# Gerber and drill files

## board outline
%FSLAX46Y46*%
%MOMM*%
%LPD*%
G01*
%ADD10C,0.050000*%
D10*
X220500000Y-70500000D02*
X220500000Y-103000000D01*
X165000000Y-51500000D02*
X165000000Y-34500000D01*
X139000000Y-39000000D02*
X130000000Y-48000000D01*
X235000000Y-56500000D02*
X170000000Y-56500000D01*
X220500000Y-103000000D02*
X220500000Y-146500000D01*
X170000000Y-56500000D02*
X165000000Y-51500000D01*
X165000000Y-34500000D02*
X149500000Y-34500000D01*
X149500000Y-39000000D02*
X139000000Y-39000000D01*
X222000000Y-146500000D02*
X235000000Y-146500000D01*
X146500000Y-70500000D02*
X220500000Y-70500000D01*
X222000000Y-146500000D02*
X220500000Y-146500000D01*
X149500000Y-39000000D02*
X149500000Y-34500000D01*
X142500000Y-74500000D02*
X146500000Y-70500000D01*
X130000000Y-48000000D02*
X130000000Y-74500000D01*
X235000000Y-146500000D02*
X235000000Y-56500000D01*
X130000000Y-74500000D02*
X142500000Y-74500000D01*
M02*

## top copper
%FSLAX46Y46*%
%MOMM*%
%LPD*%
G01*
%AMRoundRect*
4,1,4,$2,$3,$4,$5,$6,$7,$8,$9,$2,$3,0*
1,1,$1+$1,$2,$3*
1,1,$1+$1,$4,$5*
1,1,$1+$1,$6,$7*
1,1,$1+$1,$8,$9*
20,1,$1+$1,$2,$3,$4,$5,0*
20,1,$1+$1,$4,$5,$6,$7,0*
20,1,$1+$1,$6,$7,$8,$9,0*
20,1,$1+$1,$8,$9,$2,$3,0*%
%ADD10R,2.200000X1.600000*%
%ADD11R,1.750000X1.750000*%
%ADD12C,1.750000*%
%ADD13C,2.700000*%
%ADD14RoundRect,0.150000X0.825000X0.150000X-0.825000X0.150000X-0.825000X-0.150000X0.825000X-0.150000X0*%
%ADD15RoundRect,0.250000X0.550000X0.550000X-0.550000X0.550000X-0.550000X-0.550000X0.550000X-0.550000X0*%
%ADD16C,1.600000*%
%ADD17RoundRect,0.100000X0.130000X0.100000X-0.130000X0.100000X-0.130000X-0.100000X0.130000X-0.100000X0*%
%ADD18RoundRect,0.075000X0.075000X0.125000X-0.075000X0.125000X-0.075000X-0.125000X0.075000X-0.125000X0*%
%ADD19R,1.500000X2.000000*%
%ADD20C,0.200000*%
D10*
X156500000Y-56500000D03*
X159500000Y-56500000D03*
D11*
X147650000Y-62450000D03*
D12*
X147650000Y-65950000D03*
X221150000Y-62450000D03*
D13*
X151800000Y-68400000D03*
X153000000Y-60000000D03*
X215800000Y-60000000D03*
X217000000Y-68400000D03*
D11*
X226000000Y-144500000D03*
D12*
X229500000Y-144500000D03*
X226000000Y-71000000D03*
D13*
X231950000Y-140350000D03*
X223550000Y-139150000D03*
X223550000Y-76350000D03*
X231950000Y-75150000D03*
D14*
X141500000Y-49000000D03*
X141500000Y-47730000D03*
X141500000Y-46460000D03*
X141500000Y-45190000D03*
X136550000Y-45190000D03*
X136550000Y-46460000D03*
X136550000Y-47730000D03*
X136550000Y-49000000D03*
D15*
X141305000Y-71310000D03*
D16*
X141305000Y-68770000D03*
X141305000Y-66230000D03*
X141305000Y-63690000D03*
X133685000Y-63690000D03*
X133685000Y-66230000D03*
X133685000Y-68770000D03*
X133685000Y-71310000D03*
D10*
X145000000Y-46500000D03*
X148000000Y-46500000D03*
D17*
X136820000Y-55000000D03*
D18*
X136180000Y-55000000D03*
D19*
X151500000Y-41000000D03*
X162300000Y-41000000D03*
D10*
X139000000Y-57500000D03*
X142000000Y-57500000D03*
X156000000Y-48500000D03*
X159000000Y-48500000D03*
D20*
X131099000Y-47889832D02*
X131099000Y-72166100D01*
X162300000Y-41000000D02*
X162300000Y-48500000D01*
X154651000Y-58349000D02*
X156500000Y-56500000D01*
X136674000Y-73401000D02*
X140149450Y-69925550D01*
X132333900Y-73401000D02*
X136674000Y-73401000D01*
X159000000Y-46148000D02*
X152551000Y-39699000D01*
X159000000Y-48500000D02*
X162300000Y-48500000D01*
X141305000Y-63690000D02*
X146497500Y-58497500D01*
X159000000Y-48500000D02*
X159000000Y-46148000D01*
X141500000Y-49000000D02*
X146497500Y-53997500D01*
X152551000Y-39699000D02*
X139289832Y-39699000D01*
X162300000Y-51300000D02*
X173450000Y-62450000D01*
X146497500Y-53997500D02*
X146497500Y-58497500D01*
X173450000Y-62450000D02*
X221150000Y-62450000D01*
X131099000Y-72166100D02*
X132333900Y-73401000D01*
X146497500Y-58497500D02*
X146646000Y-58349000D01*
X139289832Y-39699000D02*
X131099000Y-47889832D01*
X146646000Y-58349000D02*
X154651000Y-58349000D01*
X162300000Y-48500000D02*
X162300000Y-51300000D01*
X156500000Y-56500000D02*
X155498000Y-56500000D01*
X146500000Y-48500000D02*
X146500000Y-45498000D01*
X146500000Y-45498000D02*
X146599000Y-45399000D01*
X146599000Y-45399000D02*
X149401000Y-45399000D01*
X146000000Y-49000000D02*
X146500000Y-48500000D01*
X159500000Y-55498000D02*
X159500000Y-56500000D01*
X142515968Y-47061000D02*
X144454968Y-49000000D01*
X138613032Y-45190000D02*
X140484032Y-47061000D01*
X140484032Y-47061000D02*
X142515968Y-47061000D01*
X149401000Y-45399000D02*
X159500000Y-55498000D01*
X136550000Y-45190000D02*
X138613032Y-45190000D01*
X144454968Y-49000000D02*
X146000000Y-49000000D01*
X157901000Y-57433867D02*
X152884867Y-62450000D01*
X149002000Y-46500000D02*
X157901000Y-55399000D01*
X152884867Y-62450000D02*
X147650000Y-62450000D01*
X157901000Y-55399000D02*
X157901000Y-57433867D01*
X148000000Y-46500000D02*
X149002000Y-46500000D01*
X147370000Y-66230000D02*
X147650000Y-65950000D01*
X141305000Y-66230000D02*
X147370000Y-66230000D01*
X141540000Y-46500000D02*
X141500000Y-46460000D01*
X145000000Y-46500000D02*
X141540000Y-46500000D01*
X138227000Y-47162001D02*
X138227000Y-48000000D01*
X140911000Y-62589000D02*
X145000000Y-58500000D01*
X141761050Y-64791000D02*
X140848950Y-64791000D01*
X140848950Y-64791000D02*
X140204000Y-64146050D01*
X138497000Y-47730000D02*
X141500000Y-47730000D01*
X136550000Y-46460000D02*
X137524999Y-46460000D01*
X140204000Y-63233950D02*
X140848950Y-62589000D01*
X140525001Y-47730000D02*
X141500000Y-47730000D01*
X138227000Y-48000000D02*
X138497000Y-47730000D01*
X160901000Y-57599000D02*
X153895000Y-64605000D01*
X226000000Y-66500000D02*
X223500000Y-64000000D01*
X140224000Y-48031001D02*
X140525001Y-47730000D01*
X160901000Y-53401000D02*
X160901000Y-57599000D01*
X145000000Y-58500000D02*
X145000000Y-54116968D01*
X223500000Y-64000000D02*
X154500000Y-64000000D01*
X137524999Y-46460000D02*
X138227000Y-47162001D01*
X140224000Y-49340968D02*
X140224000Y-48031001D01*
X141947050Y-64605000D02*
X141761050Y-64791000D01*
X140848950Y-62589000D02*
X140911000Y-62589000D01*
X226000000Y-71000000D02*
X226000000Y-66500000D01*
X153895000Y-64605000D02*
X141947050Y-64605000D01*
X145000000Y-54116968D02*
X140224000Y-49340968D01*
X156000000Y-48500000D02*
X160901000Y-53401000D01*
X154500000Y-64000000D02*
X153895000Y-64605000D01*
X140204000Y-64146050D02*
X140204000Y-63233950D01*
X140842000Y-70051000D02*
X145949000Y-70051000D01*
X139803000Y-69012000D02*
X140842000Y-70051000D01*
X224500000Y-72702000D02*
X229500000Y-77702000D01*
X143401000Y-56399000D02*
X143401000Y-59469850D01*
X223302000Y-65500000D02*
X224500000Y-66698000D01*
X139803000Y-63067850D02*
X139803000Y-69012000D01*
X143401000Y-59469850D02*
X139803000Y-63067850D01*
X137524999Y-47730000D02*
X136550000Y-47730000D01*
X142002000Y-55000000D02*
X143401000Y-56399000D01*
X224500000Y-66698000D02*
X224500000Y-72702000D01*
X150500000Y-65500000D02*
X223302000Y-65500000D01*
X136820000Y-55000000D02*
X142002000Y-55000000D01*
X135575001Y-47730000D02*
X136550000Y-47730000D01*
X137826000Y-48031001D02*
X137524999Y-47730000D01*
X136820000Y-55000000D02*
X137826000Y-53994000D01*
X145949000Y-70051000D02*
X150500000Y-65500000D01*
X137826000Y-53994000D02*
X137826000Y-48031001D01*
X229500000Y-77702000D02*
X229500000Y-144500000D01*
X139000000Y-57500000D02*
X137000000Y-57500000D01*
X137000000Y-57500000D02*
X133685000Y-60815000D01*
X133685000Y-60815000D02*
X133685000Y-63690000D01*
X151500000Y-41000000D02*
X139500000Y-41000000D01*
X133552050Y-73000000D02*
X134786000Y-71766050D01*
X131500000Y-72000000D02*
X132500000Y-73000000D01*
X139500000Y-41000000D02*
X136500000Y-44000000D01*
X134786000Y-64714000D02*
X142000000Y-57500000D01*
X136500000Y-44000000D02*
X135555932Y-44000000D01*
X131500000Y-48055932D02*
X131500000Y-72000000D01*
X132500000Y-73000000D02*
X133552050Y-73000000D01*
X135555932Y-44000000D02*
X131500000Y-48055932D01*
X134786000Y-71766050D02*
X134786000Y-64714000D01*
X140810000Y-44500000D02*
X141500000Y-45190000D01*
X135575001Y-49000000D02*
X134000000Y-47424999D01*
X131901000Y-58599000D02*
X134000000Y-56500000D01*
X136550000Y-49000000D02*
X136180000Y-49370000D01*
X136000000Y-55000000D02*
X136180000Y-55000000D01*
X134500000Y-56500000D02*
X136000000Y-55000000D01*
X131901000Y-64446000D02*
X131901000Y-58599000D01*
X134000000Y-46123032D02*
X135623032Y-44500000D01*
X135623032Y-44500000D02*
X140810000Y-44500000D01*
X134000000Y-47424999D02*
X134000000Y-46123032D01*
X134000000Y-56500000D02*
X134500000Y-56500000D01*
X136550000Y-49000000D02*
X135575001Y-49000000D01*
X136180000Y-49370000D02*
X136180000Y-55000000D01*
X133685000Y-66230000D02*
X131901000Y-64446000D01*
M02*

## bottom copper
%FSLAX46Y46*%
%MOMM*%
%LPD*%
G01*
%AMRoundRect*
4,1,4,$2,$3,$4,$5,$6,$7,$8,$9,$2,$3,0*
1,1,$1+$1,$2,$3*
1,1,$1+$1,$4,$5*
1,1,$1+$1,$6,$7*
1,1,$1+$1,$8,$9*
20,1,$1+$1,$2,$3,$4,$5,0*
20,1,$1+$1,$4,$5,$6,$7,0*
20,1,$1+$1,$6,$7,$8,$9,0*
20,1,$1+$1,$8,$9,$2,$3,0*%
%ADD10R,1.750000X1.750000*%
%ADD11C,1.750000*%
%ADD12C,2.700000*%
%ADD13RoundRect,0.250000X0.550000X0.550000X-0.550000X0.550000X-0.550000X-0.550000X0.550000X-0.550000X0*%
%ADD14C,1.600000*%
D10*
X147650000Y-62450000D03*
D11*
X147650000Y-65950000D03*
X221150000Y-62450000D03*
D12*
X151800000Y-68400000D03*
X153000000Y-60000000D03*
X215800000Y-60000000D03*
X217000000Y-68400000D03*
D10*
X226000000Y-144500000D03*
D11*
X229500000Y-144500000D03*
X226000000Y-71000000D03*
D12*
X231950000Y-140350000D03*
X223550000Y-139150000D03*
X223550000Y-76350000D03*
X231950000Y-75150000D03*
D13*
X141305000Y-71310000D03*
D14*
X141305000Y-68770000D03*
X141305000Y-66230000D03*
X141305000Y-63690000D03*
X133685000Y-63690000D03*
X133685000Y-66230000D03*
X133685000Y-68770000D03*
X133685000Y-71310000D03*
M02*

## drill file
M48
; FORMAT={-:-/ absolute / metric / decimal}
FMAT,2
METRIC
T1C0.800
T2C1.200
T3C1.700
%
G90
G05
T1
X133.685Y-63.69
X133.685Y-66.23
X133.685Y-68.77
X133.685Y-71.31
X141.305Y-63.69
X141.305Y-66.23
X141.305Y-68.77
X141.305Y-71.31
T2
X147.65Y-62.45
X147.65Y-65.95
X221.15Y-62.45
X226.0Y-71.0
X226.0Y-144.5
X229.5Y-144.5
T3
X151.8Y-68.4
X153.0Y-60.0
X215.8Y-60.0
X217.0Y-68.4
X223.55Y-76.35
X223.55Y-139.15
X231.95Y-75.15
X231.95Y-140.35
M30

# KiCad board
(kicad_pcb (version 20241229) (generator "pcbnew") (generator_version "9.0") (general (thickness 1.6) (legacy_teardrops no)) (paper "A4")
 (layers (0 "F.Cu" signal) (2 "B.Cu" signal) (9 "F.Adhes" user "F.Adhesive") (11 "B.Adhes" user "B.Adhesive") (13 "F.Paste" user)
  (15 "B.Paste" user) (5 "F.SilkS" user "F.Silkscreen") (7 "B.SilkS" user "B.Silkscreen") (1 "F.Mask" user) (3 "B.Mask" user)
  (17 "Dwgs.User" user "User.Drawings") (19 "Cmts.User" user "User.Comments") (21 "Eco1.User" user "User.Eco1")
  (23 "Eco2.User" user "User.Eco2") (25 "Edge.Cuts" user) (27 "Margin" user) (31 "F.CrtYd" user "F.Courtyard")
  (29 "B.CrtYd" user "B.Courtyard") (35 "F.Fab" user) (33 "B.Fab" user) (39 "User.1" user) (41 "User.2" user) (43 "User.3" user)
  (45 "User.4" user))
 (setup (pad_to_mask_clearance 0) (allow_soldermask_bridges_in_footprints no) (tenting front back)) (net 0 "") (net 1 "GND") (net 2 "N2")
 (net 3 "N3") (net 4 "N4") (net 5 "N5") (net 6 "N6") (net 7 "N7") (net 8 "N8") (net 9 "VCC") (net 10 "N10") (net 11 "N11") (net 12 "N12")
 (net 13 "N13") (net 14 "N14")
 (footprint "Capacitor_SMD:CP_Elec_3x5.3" (layer "F.Cu") (at 158 56.5)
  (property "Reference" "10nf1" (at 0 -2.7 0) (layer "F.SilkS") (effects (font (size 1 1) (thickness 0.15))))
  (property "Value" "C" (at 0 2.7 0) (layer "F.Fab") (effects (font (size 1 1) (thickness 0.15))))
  (pad "1" smd rect (at -1.5 0) (size 2.2 1.6) (layers "F.Cu" "F.Mask" "F.Paste") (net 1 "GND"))
  (pad "2" smd rect (at 1.5 0) (size 2.2 1.6) (layers "F.Cu" "F.Mask" "F.Paste") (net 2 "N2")))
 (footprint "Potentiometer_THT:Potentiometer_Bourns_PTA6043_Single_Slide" (layer "F.Cu") (at 147.65 62.45)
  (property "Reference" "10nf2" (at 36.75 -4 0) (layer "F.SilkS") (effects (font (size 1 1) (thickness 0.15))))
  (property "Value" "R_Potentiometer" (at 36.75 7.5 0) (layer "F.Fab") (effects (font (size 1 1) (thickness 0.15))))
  (pad "1" thru_hole rect (at 0 0) (size 1.75 1.75) (drill 1.2) (layers "*.Cu" "*.Mask") (remove_unused_layers no) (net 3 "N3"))
  (pad "2" thru_hole circle (at 0 3.5) (size 1.75 1.75) (drill 1.2) (layers "*.Cu" "*.Mask") (remove_unused_layers no) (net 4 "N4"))
  (pad "3" thru_hole circle (at 73.5 0) (size 1.75 1.75) (drill 1.2) (layers "*.Cu" "*.Mask") (remove_unused_layers no) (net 1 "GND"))
  (pad "MP" thru_hole circle (at 4.15 5.95) (size 2.7 2.7) (drill 1.7) (layers "*.Cu" "*.Mask") (remove_unused_layers no))
  (pad "MP" thru_hole circle (at 5.35 -2.45) (size 2.7 2.7) (drill 1.7) (layers "*.Cu" "*.Mask") (remove_unused_layers no))
  (pad "MP" thru_hole circle (at 68.15 -2.45) (size 2.7 2.7) (drill 1.7) (layers "*.Cu" "*.Mask") (remove_unused_layers no))
  (pad "MP" thru_hole circle (at 69.35 5.95) (size 2.7 2.7) (drill 1.7) (layers "*.Cu" "*.Mask") (remove_unused_layers no)))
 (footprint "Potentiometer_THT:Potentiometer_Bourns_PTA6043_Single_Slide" (layer "F.Cu") (at 226 144.5 90)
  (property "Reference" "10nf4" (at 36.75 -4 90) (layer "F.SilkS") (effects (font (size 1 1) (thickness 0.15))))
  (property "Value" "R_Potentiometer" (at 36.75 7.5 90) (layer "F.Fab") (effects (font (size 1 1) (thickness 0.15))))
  (pad "1" thru_hole rect (at 0 0 90) (size 1.75 1.75) (drill 1.2) (layers "*.Cu" "*.Mask") (remove_unused_layers no) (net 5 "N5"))
  (pad "2" thru_hole circle (at 0 3.5 90) (size 1.75 1.75) (drill 1.2) (layers "*.Cu" "*.Mask") (remove_unused_layers no) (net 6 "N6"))
  (pad "3" thru_hole circle (at 73.5 0 90) (size 1.75 1.75) (drill 1.2) (layers "*.Cu" "*.Mask") (remove_unused_layers no) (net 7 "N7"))
  (pad "MP" thru_hole circle (at 4.15 5.95 90) (size 2.7 2.7) (drill 1.7) (layers "*.Cu" "*.Mask") (remove_unused_layers no))
  (pad "MP" thru_hole circle (at 5.35 -2.45 90) (size 2.7 2.7) (drill 1.7) (layers "*.Cu" "*.Mask") (remove_unused_layers no))
  (pad "MP" thru_hole circle (at 68.15 -2.45 90) (size 2.7 2.7) (drill 1.7) (layers "*.Cu" "*.Mask") (remove_unused_layers no))
  (pad "MP" thru_hole circle (at 69.35 5.95 90) (size 2.7 2.7) (drill 1.7) (layers "*.Cu" "*.Mask") (remove_unused_layers no)))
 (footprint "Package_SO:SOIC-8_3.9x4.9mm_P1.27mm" (layer "F.Cu") (at 139.025 47.095 180)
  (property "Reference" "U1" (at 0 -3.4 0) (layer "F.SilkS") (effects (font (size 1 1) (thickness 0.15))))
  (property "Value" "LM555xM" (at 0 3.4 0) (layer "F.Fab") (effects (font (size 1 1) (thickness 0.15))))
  (pad "1" smd roundrect (at -2.475 -1.905 180) (size 1.95 0.6) (layers "F.Cu" "F.Mask" "F.Paste") (roundrect_rratio 0.25) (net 1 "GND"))
  (pad "2" smd roundrect (at -2.475 -0.635 180) (size 1.95 0.6) (layers "F.Cu" "F.Mask" "F.Paste") (roundrect_rratio 0.25) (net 7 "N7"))
  (pad "3" smd roundrect (at -2.475 0.635 180) (size 1.95 0.6) (layers "F.Cu" "F.Mask" "F.Paste") (roundrect_rratio 0.25) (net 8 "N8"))
  (pad "4" smd roundrect (at -2.475 1.905 180) (size 1.95 0.6) (layers "F.Cu" "F.Mask" "F.Paste") (roundrect_rratio 0.25) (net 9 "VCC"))
  (pad "5" smd roundrect (at 2.475 1.905 180) (size 1.95 0.6) (layers "F.Cu" "F.Mask" "F.Paste") (roundrect_rratio 0.25) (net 2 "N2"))
  (pad "6" smd roundrect (at 2.475 0.635 180) (size 1.95 0.6) (layers "F.Cu" "F.Mask" "F.Paste") (roundrect_rratio 0.25) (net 7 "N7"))
  (pad "7" smd roundrect (at 2.475 -0.635 180) (size 1.95 0.6) (layers "F.Cu" "F.Mask" "F.Paste") (roundrect_rratio 0.25) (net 6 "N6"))
  (pad "8" smd roundrect (at 2.475 -1.905 180) (size 1.95 0.6) (layers "F.Cu" "F.Mask" "F.Paste") (roundrect_rratio 0.25) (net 9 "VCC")))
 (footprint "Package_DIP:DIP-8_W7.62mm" (layer "F.Cu") (at 141.305 71.31 180)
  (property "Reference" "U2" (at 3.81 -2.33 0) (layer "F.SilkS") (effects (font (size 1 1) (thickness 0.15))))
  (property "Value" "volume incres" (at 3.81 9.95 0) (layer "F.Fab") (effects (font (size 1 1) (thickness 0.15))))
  (pad "1" thru_hole roundrect (at 0 0 180) (size 1.6 1.6) (drill 0.8) (layers "*.Cu" "*.Mask") (remove_unused_layers no)
   (roundrect_rratio 0.15625) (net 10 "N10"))
  (pad "2" thru_hole circle (at 0 2.54 180) (size 1.6 1.6) (drill 0.8) (layers "*.Cu" "*.Mask") (remove_unused_layers no) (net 1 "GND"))
  (pad "3" thru_hole circle (at 0 5.08 180) (size 1.6 1.6) (drill 0.8) (layers "*.Cu" "*.Mask") (remove_unused_layers no) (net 4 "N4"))
  (pad "4" thru_hole circle (at 0 7.62 180) (size 1.6 1.6) (drill 0.8) (layers "*.Cu" "*.Mask") (remove_unused_layers no) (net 1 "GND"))
  (pad "5" thru_hole circle (at 7.62 7.62 180) (size 1.6 1.6) (drill 0.8) (layers "*.Cu" "*.Mask") (remove_unused_layers no) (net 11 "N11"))
  (pad "6" thru_hole circle (at 7.62 5.08 180) (size 1.6 1.6) (drill 0.8) (layers "*.Cu" "*.Mask") (remove_unused_layers no) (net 9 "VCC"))
  (pad "7" thru_hole circle (at 7.62 2.54 180) (size 1.6 1.6) (drill 0.8) (layers "*.Cu" "*.Mask") (remove_unused_layers no) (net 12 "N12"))
  (pad "8" thru_hole circle (at 7.62 0 180) (size 1.6 1.6) (drill 0.8) (layers "*.Cu" "*.Mask") (remove_unused_layers no) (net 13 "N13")))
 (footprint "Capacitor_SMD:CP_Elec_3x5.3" (layer "F.Cu") (at 146.5 46.5)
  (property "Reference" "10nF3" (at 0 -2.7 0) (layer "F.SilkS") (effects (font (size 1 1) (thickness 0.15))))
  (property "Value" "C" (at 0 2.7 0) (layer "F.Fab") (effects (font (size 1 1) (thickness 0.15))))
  (pad "1" smd rect (at -1.5 0) (size 2.2 1.6) (layers "F.Cu" "F.Mask" "F.Paste") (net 8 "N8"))
  (pad "2" smd rect (at 1.5 0) (size 2.2 1.6) (layers "F.Cu" "F.Mask" "F.Paste") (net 3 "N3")))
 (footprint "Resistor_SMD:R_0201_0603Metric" (layer "F.Cu") (at 136.5 55 180)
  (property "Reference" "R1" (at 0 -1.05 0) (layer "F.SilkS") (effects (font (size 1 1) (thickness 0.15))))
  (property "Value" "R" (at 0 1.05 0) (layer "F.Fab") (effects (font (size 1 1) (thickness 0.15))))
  (pad "" smd roundrect (at -0.345 0 180) (size 0.318 0.36) (layers "F.Paste") (roundrect_rratio 0.25))
  (pad "" smd roundrect (at 0.345 0 180) (size 0.318 0.36) (layers "F.Paste") (roundrect_rratio 0.25))
  (pad "1" smd roundrect (at -0.32 0 180) (size 0.46 0.4) (layers "F.Cu" "F.Mask") (roundrect_rratio 0.25) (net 6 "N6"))
  (pad "2" smd roundrect (at 0.32 0 180) (size 0.3 0.4) (layers "F.Cu" "F.Mask") (roundrect_rratio 0.25) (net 9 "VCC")))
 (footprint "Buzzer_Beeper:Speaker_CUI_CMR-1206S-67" (layer "F.Cu") (at 156.9 38.7)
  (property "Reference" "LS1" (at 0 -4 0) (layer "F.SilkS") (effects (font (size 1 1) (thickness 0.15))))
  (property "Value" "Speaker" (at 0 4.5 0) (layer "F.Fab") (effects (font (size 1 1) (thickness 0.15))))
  (pad "1" smd rect (at -5.4 2.3 180) (size 1.5 2) (layers "F.Cu" "F.Mask") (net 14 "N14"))
  (pad "2" smd rect (at 5.4 2.3 180) (size 1.5 2) (layers "F.Cu" "F.Mask") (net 1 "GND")))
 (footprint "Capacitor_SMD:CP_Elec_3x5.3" (layer "F.Cu") (at 140.5 57.5)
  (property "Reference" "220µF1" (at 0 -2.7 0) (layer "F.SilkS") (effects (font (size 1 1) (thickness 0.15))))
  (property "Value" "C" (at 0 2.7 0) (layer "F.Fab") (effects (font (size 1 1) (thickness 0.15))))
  (pad "1" smd rect (at -1.5 0) (size 2.2 1.6) (layers "F.Cu" "F.Mask" "F.Paste") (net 11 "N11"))
  (pad "2" smd rect (at 1.5 0) (size 2.2 1.6) (layers "F.Cu" "F.Mask" "F.Paste") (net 14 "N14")))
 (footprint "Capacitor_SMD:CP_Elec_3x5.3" (layer "F.Cu") (at 157.5 48.5)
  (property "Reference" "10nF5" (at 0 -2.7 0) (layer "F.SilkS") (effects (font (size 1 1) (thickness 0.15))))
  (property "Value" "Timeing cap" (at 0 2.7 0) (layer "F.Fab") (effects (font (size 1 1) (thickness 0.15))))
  (pad "1" smd rect (at -1.5 0) (size 2.2 1.6) (layers "F.Cu" "F.Mask" "F.Paste") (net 7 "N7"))
  (pad "2" smd rect (at 1.5 0) (size 2.2 1.6) (layers "F.Cu" "F.Mask" "F.Paste") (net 1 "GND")))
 (gr_line (start 220.5 70.5) (end 220.5 103) (stroke (width 0.05) (type default)) (layer "Edge.Cuts"))
 (gr_line (start 165 51.5) (end 165 34.5) (stroke (width 0.05) (type default)) (layer "Edge.Cuts"))
 (gr_line (start 139 39) (end 130 48) (stroke (width 0.05) (type default)) (layer "Edge.Cuts"))
 (gr_line (start 235 56.5) (end 170 56.5) (stroke (width 0.05) (type default)) (layer "Edge.Cuts"))
 (gr_line (start 220.5 103) (end 220.5 146.5) (stroke (width 0.05) (type default)) (layer "Edge.Cuts"))
 (gr_line (start 170 56.5) (end 165 51.5) (stroke (width 0.05) (type default)) (layer "Edge.Cuts"))
 (gr_line (start 165 34.5) (end 149.5 34.5) (stroke (width 0.05) (type default)) (layer "Edge.Cuts"))
 (gr_line (start 149.5 39) (end 139 39) (stroke (width 0.05) (type default)) (layer "Edge.Cuts"))
 (gr_line (start 222 146.5) (end 235 146.5) (stroke (width 0.05) (type default)) (layer "Edge.Cuts"))
 (gr_line (start 146.5 70.5) (end 220.5 70.5) (stroke (width 0.05) (type default)) (layer "Edge.Cuts"))
 (gr_line (start 222 146.5) (end 220.5 146.5) (stroke (width 0.05) (type default)) (layer "Edge.Cuts"))
 (gr_line (start 149.5 39) (end 149.5 34.5) (stroke (width 0.05) (type default)) (layer "Edge.Cuts"))
 (gr_line (start 142.5 74.5) (end 146.5 70.5) (stroke (width 0.05) (type default)) (layer "Edge.Cuts"))
 (gr_line (start 130 48) (end 130 74.5) (stroke (width 0.05) (type default)) (layer "Edge.Cuts"))
 (gr_line (start 235 146.5) (end 235 56.5) (stroke (width 0.05) (type default)) (layer "Edge.Cuts"))
 (gr_line (start 130 74.5) (end 142.5 74.5) (stroke (width 0.05) (type default)) (layer "Edge.Cuts"))
 (segment (start 131.099 47.889832) (end 131.099 72.1661) (width 0.2) (layer "F.Cu") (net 1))
 (segment (start 162.3 41) (end 162.3 48.5) (width 0.2) (layer "F.Cu") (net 1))
 (segment (start 154.651 58.349) (end 156.5 56.5) (width 0.2) (layer "F.Cu") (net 1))
 (segment (start 136.674 73.401) (end 140.14945 69.92555) (width 0.2) (layer "F.Cu") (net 1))
 (segment (start 132.3339 73.401) (end 136.674 73.401) (width 0.2) (layer "F.Cu") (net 1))
 (segment (start 159 46.148) (end 152.551 39.699) (width 0.2) (layer "F.Cu") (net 1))
 (segment (start 159 48.5) (end 162.3 48.5) (width 0.2) (layer "F.Cu") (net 1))
 (segment (start 141.305 63.69) (end 146.4975 58.4975) (width 0.2) (layer "F.Cu") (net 1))
 (segment (start 159 48.5) (end 159 46.148) (width 0.2) (layer "F.Cu") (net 1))
 (segment (start 141.5 49) (end 146.4975 53.9975) (width 0.2) (layer "F.Cu") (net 1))
 (segment (start 152.551 39.699) (end 139.289832 39.699) (width 0.2) (layer "F.Cu") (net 1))
 (segment (start 162.3 51.3) (end 173.45 62.45) (width 0.2) (layer "F.Cu") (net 1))
 (segment (start 146.4975 53.9975) (end 146.4975 58.4975) (width 0.2) (layer "F.Cu") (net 1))
 (segment (start 173.45 62.45) (end 221.15 62.45) (width 0.2) (layer "F.Cu") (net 1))
 (segment (start 131.099 72.1661) (end 132.3339 73.401) (width 0.2) (layer "F.Cu") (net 1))
 (segment (start 146.4975 58.4975) (end 146.646 58.349) (width 0.2) (layer "F.Cu") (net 1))
 (segment (start 139.289832 39.699) (end 131.099 47.889832) (width 0.2) (layer "F.Cu") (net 1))
 (segment (start 146.646 58.349) (end 154.651 58.349) (width 0.2) (layer "F.Cu") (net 1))
 (segment (start 162.3 48.5) (end 162.3 51.3) (width 0.2) (layer "F.Cu") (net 1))
 (segment (start 156.5 56.5) (end 155.498 56.5) (width 0.2) (layer "F.Cu") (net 1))
 (segment (start 146.5 48.5) (end 146.5 45.498) (width 0.2) (layer "F.Cu") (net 2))
 (segment (start 146.5 45.498) (end 146.599 45.399) (width 0.2) (layer "F.Cu") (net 2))
 (segment (start 146.599 45.399) (end 149.401 45.399) (width 0.2) (layer "F.Cu") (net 2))
 (segment (start 146 49) (end 146.5 48.5) (width 0.2) (layer "F.Cu") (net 2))
 (segment (start 159.5 55.498) (end 159.5 56.5) (width 0.2) (layer "F.Cu") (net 2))
 (segment (start 142.515968 47.061) (end 144.454968 49) (width 0.2) (layer "F.Cu") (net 2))
 (segment (start 138.613032 45.19) (end 140.484032 47.061) (width 0.2) (layer "F.Cu") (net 2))
 (segment (start 140.484032 47.061) (end 142.515968 47.061) (width 0.2) (layer "F.Cu") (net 2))
 (segment (start 149.401 45.399) (end 159.5 55.498) (width 0.2) (layer "F.Cu") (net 2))
 (segment (start 136.55 45.19) (end 138.613032 45.19) (width 0.2) (layer "F.Cu") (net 2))
 (segment (start 144.454968 49) (end 146 49) (width 0.2) (layer "F.Cu") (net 2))
 (segment (start 157.901 57.433867) (end 152.884867 62.45) (width 0.2) (layer "F.Cu") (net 3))
 (segment (start 149.002 46.5) (end 157.901 55.399) (width 0.2) (layer "F.Cu") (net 3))
 (segment (start 152.884867 62.45) (end 147.65 62.45) (width 0.2) (layer "F.Cu") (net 3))
 (segment (start 157.901 55.399) (end 157.901 57.433867) (width 0.2) (layer "F.Cu") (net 3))
 (segment (start 148 46.5) (end 149.002 46.5) (width 0.2) (layer "F.Cu") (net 3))
 (segment (start 147.37 66.23) (end 147.65 65.95) (width 0.2) (layer "F.Cu") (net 4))
 (segment (start 141.305 66.23) (end 147.37 66.23) (width 0.2) (layer "F.Cu") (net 4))
 (segment (start 141.54 46.5) (end 141.5 46.46) (width 0.2) (layer "F.Cu") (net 8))
 (segment (start 145 46.5) (end 141.54 46.5) (width 0.2) (layer "F.Cu") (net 8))
 (segment (start 138.227 47.162001) (end 138.227 48) (width 0.2) (layer "F.Cu") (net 7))
 (segment (start 140.911 62.589) (end 145 58.5) (width 0.2) (layer "F.Cu") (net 7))
 (segment (start 141.76105 64.791) (end 140.84895 64.791) (width 0.2) (layer "F.Cu") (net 7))
 (segment (start 140.84895 64.791) (end 140.204 64.14605) (width 0.2) (layer "F.Cu") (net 7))
 (segment (start 138.497 47.73) (end 141.5 47.73) (width 0.2) (layer "F.Cu") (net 7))
 (segment (start 136.55 46.46) (end 137.524999 46.46) (width 0.2) (layer "F.Cu") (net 7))
 (segment (start 140.204 63.23395) (end 140.84895 62.589) (width 0.2) (layer "F.Cu") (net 7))
 (segment (start 140.525001 47.73) (end 141.5 47.73) (width 0.2) (layer "F.Cu") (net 7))
 (segment (start 138.227 48) (end 138.497 47.73) (width 0.2) (layer "F.Cu") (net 7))
 (segment (start 160.901 57.599) (end 153.895 64.605) (width 0.2) (layer "F.Cu") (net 7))
 (segment (start 226 66.5) (end 223.5 64) (width 0.2) (layer "F.Cu") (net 7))
 (segment (start 140.224 48.031001) (end 140.525001 47.73) (width 0.2) (layer "F.Cu") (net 7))
 (segment (start 160.901 53.401) (end 160.901 57.599) (width 0.2) (layer "F.Cu") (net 7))
 (segment (start 145 58.5) (end 145 54.116968) (width 0.2) (layer "F.Cu") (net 7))
 (segment (start 223.5 64) (end 154.5 64) (width 0.2) (layer "F.Cu") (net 7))
 (segment (start 137.524999 46.46) (end 138.227 47.162001) (width 0.2) (layer "F.Cu") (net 7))
 (segment (start 140.224 49.340968) (end 140.224 48.031001) (width 0.2) (layer "F.Cu") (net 7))
 (segment (start 141.94705 64.605) (end 141.76105 64.791) (width 0.2) (layer "F.Cu") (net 7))
 (segment (start 140.84895 62.589) (end 140.911 62.589) (width 0.2) (layer "F.Cu") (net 7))
 (segment (start 226 71) (end 226 66.5) (width 0.2) (layer "F.Cu") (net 7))
 (segment (start 153.895 64.605) (end 141.94705 64.605) (width 0.2) (layer "F.Cu") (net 7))
 (segment (start 145 54.116968) (end 140.224 49.340968) (width 0.2) (layer "F.Cu") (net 7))
 (segment (start 156 48.5) (end 160.901 53.401) (width 0.2) (layer "F.Cu") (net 7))
 (segment (start 154.5 64) (end 153.895 64.605) (width 0.2) (layer "F.Cu") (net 7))
 (segment (start 140.204 64.14605) (end 140.204 63.23395) (width 0.2) (layer "F.Cu") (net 7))
 (segment (start 140.842 70.051) (end 145.949 70.051) (width 0.2) (layer "F.Cu") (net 6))
 (segment (start 139.803 69.012) (end 140.842 70.051) (width 0.2) (layer "F.Cu") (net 6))
 (segment (start 224.5 72.702) (end 229.5 77.702) (width 0.2) (layer "F.Cu") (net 6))
 (segment (start 143.401 56.399) (end 143.401 59.46985) (width 0.2) (layer "F.Cu") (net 6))
 (segment (start 223.302 65.5) (end 224.5 66.698) (width 0.2) (layer "F.Cu") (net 6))
 (segment (start 139.803 63.06785) (end 139.803 69.012) (width 0.2) (layer "F.Cu") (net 6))
 (segment (start 143.401 59.46985) (end 139.803 63.06785) (width 0.2) (layer "F.Cu") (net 6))
 (segment (start 137.524999 47.73) (end 136.55 47.73) (width 0.2) (layer "F.Cu") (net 6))
 (segment (start 142.002 55) (end 143.401 56.399) (width 0.2) (layer "F.Cu") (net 6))
 (segment (start 224.5 66.698) (end 224.5 72.702) (width 0.2) (layer "F.Cu") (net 6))
 (segment (start 150.5 65.5) (end 223.302 65.5) (width 0.2) (layer "F.Cu") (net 6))
 (segment (start 136.82 55) (end 142.002 55) (width 0.2) (layer "F.Cu") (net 6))
 (segment (start 135.575001 47.73) (end 136.55 47.73) (width 0.2) (layer "F.Cu") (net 6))
 (segment (start 137.826 48.031001) (end 137.524999 47.73) (width 0.2) (layer "F.Cu") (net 6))
 (segment (start 136.82 55) (end 137.826 53.994) (width 0.2) (layer "F.Cu") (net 6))
 (segment (start 145.949 70.051) (end 150.5 65.5) (width 0.2) (layer "F.Cu") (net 6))
 (segment (start 137.826 53.994) (end 137.826 48.031001) (width 0.2) (layer "F.Cu") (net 6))
 (segment (start 229.5 77.702) (end 229.5 144.5) (width 0.2) (layer "F.Cu") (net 6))
 (segment (start 139 57.5) (end 137 57.5) (width 0.2) (layer "F.Cu") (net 11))
 (segment (start 137 57.5) (end 133.685 60.815) (width 0.2) (layer "F.Cu") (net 11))
 (segment (start 133.685 60.815) (end 133.685 63.69) (width 0.2) (layer "F.Cu") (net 11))
 (segment (start 151.5 41) (end 139.5 41) (width 0.2) (layer "F.Cu") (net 14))
 (segment (start 133.55205 73) (end 134.786 71.76605) (width 0.2) (layer "F.Cu") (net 14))
 (segment (start 131.5 72) (end 132.5 73) (width 0.2) (layer "F.Cu") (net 14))
 (segment (start 139.5 41) (end 136.5 44) (width 0.2) (layer "F.Cu") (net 14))
 (segment (start 134.786 64.714) (end 142 57.5) (width 0.2) (layer "F.Cu") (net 14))
 (segment (start 136.5 44) (end 135.555932 44) (width 0.2) (layer "F.Cu") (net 14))
 (segment (start 131.5 48.055932) (end 131.5 72) (width 0.2) (layer "F.Cu") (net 14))
 (segment (start 132.5 73) (end 133.55205 73) (width 0.2) (layer "F.Cu") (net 14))
 (segment (start 135.555932 44) (end 131.5 48.055932) (width 0.2) (layer "F.Cu") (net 14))
 (segment (start 134.786 71.76605) (end 134.786 64.714) (width 0.2) (layer "F.Cu") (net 14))
 (segment (start 140.81 44.5) (end 141.5 45.19) (width 0.2) (layer "F.Cu") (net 9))
 (segment (start 135.575001 49) (end 134 47.424999) (width 0.2) (layer "F.Cu") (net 9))
 (segment (start 131.901 58.599) (end 134 56.5) (width 0.2) (layer "F.Cu") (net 9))
 (segment (start 136.55 49) (end 136.18 49.37) (width 0.2) (layer "F.Cu") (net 9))
 (segment (start 136 55) (end 136.18 55) (width 0.2) (layer "F.Cu") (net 9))
 (segment (start 134.5 56.5) (end 136 55) (width 0.2) (layer "F.Cu") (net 9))
 (segment (start 131.901 64.446) (end 131.901 58.599) (width 0.2) (layer "F.Cu") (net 9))
 (segment (start 134 46.123032) (end 135.623032 44.5) (width 0.2) (layer "F.Cu") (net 9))
 (segment (start 135.623032 44.5) (end 140.81 44.5) (width 0.2) (layer "F.Cu") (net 9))
 (segment (start 134 47.424999) (end 134 46.123032) (width 0.2) (layer "F.Cu") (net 9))
 (segment (start 134 56.5) (end 134.5 56.5) (width 0.2) (layer "F.Cu") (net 9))
 (segment (start 136.55 49) (end 135.575001 49) (width 0.2) (layer "F.Cu") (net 9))
 (segment (start 136.18 49.37) (end 136.18 55) (width 0.2) (layer "F.Cu") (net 9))
 (segment (start 133.685 66.23) (end 131.901 64.446) (width 0.2) (layer "F.Cu") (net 9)))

